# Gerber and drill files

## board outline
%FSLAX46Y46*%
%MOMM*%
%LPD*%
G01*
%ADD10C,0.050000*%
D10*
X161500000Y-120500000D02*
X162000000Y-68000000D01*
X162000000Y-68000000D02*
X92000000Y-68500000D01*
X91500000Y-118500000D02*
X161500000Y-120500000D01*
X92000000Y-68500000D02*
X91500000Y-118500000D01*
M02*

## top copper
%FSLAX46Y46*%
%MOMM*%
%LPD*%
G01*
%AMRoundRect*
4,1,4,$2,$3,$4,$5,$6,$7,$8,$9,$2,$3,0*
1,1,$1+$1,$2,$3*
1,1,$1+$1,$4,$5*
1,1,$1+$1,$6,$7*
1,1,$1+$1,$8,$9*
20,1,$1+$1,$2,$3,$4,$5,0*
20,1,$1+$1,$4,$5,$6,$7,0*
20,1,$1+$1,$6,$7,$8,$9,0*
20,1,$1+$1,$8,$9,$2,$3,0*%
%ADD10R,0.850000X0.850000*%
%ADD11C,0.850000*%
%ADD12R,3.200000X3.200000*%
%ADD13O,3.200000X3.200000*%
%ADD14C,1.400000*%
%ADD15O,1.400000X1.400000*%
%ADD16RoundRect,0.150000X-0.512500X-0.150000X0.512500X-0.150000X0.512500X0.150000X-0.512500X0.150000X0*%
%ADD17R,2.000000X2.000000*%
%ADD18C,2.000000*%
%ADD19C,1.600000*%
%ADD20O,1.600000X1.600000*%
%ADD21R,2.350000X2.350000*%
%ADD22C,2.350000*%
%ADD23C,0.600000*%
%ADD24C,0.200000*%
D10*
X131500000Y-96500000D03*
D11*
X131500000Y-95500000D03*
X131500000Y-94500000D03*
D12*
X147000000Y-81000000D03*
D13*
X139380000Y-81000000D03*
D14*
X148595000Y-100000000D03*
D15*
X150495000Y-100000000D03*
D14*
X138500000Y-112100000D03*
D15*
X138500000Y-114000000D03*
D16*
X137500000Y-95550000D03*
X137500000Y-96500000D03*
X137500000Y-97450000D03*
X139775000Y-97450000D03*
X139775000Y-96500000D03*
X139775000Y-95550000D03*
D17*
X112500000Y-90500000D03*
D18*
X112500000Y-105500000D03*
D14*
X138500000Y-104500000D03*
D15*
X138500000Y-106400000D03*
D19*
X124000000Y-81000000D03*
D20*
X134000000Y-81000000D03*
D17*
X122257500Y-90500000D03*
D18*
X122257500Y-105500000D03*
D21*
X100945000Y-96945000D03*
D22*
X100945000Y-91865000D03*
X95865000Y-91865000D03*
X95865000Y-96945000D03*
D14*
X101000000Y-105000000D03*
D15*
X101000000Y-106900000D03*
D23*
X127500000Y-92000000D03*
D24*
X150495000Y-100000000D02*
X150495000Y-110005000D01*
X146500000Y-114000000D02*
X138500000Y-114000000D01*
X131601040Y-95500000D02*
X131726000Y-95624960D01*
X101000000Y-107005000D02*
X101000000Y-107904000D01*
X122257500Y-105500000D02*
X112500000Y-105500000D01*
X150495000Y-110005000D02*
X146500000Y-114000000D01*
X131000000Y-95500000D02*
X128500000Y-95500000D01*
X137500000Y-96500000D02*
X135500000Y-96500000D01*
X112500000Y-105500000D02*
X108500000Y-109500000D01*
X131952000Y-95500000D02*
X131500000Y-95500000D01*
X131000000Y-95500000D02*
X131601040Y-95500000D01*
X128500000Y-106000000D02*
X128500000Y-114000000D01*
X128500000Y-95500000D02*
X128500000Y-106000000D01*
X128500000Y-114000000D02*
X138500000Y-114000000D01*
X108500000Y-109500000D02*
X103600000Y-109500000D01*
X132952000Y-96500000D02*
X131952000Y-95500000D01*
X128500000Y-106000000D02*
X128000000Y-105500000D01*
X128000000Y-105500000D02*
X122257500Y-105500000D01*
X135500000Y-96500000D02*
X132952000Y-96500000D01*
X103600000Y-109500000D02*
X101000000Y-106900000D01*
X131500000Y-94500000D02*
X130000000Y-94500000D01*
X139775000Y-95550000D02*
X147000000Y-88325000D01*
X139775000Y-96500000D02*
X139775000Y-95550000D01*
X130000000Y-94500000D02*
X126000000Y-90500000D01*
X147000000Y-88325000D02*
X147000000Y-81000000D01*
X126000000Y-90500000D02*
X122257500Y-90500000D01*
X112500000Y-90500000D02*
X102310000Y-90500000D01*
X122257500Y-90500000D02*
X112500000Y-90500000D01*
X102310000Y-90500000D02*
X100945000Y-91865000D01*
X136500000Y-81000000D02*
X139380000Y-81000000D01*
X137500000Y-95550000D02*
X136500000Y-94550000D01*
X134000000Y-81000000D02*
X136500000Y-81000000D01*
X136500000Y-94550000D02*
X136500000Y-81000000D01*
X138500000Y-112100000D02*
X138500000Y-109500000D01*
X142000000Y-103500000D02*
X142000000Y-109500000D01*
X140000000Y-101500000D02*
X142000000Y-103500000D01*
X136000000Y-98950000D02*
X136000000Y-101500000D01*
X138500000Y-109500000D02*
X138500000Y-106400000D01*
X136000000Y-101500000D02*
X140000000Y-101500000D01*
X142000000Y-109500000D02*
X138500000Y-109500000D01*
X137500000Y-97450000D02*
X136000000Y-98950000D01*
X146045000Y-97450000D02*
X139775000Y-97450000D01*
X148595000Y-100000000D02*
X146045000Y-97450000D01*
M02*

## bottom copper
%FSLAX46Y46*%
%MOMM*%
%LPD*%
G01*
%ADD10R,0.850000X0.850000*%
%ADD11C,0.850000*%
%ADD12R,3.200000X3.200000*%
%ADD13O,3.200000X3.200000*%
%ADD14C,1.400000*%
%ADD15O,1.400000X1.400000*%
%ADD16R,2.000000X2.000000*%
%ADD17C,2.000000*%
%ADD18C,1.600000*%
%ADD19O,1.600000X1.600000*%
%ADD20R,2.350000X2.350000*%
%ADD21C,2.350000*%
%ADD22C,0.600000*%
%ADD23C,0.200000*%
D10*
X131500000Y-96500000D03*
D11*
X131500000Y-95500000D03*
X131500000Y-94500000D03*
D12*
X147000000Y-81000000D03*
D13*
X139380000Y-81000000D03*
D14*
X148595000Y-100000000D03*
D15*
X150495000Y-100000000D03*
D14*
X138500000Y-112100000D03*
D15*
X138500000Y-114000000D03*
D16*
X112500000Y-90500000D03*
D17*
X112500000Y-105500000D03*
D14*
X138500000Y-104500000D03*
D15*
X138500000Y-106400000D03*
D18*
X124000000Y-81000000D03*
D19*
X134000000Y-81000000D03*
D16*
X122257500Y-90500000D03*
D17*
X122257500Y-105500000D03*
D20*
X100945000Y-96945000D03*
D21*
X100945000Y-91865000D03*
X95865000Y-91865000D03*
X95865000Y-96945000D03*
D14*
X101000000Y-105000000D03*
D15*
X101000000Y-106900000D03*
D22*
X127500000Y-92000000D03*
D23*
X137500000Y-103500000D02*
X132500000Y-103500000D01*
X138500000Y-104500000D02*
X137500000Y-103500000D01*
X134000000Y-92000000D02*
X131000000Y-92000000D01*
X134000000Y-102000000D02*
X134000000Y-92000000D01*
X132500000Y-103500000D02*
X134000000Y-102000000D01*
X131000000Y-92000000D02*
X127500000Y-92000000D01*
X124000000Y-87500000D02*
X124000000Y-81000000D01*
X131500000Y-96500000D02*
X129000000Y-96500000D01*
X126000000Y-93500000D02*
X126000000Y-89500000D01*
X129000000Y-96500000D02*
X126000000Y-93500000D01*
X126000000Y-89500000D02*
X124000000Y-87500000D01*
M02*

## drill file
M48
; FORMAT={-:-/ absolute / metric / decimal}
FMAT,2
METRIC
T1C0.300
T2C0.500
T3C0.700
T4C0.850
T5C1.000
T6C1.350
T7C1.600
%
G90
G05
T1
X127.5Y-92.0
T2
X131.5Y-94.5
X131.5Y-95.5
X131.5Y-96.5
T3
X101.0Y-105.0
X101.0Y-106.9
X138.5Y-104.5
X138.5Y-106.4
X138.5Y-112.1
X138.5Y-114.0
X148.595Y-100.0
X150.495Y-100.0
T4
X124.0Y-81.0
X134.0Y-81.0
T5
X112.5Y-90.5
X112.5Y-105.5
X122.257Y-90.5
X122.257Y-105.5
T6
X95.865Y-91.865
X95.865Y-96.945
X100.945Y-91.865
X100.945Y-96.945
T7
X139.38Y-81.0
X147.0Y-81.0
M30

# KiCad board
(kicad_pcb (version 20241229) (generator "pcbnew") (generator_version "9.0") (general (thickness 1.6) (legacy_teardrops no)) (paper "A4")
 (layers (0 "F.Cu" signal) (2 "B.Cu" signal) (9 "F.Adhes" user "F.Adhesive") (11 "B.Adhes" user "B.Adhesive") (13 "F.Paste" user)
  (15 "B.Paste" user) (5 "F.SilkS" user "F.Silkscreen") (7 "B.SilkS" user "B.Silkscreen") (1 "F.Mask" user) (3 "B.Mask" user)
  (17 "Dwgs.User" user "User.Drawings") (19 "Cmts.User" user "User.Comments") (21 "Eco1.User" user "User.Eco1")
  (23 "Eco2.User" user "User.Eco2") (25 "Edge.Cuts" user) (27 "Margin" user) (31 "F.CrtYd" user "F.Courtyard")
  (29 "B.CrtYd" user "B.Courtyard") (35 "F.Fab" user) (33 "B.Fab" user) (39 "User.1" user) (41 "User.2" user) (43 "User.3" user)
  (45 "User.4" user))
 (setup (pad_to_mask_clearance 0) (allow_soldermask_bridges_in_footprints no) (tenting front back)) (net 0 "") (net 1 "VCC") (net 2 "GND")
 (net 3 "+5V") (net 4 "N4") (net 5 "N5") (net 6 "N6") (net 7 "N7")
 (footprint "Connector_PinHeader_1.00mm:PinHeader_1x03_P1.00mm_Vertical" (layer "F.Cu") (at 131.5 96.5 180)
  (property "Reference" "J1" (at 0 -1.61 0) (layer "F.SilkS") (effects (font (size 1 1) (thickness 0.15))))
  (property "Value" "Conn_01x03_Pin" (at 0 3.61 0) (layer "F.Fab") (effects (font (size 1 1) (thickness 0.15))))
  (pad "1" thru_hole rect (at 0 0 180) (size 0.85 0.85) (drill 0.5) (layers "*.Cu" "*.Mask") (remove_unused_layers no) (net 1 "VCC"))
  (pad "2" thru_hole circle (at 0 1 180) (size 0.85 0.85) (drill 0.5) (layers "*.Cu" "*.Mask") (remove_unused_layers no) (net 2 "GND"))
  (pad "3" thru_hole circle (at 0 2 180) (size 0.85 0.85) (drill 0.5) (layers "*.Cu" "*.Mask") (remove_unused_layers no) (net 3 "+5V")))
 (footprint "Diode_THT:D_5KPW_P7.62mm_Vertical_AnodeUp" (layer "F.Cu") (at 147 81 180)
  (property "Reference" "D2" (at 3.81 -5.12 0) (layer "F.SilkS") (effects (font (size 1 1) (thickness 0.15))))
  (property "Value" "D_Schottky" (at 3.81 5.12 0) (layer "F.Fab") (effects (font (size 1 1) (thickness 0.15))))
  (pad "1" thru_hole rect (at 0 0 180) (size 3.2 3.2) (drill 1.6) (layers "*.Cu" "*.Mask") (remove_unused_layers no) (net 3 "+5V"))
  (pad "2" thru_hole oval (at 7.62 0 180) (size 3.2 3.2) (drill 1.6) (layers "*.Cu" "*.Mask") (remove_unused_layers no) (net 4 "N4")))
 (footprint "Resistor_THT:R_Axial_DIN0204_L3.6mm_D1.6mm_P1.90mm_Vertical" (layer "F.Cu") (at 148.595 100)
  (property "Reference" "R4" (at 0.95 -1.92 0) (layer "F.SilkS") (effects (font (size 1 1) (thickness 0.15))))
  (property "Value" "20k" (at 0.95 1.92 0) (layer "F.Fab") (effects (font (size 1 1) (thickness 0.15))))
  (pad "1" thru_hole circle (at 0 0) (size 1.4 1.4) (drill 0.7) (layers "*.Cu" "*.Mask") (remove_unused_layers no) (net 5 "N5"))
  (pad "2" thru_hole oval (at 1.9 0) (size 1.4 1.4) (drill 0.7) (layers "*.Cu" "*.Mask") (remove_unused_layers no) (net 2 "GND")))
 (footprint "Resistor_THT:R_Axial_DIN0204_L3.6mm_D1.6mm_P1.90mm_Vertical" (layer "F.Cu") (at 138.5 112.1 -90)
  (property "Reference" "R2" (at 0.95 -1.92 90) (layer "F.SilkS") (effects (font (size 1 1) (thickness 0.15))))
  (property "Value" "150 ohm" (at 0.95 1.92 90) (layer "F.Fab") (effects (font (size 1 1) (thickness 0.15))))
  (pad "1" thru_hole circle (at 0 0 270) (size 1.4 1.4) (drill 0.7) (layers "*.Cu" "*.Mask") (remove_unused_layers no) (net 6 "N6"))
  (pad "2" thru_hole oval (at 1.9 0 270) (size 1.4 1.4) (drill 0.7) (layers "*.Cu" "*.Mask") (remove_unused_layers no) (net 2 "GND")))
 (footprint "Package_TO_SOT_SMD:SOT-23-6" (layer "F.Cu") (at 138.6375 96.5)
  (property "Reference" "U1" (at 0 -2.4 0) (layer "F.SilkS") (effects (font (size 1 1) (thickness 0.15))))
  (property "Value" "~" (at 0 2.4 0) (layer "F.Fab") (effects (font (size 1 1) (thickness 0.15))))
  (pad "1" smd roundrect (at -1.1375 -0.95) (size 1.325 0.6) (layers "F.Cu" "F.Mask" "F.Paste") (roundrect_rratio 0.25) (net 4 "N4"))
  (pad "2" smd roundrect (at -1.1375 0) (size 1.325 0.6) (layers "F.Cu" "F.Mask" "F.Paste") (roundrect_rratio 0.25) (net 2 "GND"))
  (pad "3" smd roundrect (at -1.1375 0.95) (size 1.325 0.6) (layers "F.Cu" "F.Mask" "F.Paste") (roundrect_rratio 0.25) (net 6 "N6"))
  (pad "4" smd roundrect (at 1.1375 0.95) (size 1.325 0.6) (layers "F.Cu" "F.Mask" "F.Paste") (roundrect_rratio 0.25) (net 5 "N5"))
  (pad "5" smd roundrect (at 1.1375 0) (size 1.325 0.6) (layers "F.Cu" "F.Mask" "F.Paste") (roundrect_rratio 0.25) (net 3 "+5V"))
  (pad "6" smd roundrect (at 1.1375 -0.95) (size 1.325 0.6) (layers "F.Cu" "F.Mask" "F.Paste") (roundrect_rratio 0.25) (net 3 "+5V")))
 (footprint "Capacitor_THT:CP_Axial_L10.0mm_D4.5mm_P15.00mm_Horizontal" (layer "F.Cu") (at 112.5 90.5 -90)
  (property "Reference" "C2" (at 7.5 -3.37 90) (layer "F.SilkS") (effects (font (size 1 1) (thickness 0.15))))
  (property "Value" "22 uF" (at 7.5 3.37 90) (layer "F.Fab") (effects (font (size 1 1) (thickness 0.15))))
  (pad "1" thru_hole rect (at 0 0 270) (size 2 2) (drill 1) (layers "*.Cu" "*.Mask") (remove_unused_layers no) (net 3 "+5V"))
  (pad "2" thru_hole circle (at 15 0 270) (size 2 2) (drill 1) (layers "*.Cu" "*.Mask") (remove_unused_layers no) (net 2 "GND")))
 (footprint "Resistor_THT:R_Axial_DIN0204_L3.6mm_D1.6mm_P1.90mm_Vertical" (layer "F.Cu") (at 138.5 104.5 -90)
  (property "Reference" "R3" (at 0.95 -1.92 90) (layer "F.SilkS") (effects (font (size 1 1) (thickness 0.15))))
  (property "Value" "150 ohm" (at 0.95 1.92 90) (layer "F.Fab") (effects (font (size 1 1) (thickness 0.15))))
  (pad "1" thru_hole circle (at 0 0 270) (size 1.4 1.4) (drill 0.7) (layers "*.Cu" "*.Mask") (remove_unused_layers no) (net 3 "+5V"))
  (pad "2" thru_hole oval (at 1.9 0 270) (size 1.4 1.4) (drill 0.7) (layers "*.Cu" "*.Mask") (remove_unused_layers no) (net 6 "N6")))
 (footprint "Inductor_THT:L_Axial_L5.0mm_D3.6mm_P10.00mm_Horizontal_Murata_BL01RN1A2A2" (layer "F.Cu") (at 124 81)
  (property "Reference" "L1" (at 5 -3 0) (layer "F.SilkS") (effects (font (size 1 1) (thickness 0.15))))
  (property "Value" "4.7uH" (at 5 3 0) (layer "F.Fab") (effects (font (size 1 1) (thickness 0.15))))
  (pad "1" thru_hole circle (at 0 0) (size 1.6 1.6) (drill 0.85) (layers "*.Cu" "*.Mask") (remove_unused_layers no) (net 1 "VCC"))
  (pad "2" thru_hole oval (at 10 0) (size 1.6 1.6) (drill 0.85) (layers "*.Cu" "*.Mask") (remove_unused_layers no) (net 4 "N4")))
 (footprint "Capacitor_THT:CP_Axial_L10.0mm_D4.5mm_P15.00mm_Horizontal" (layer "F.Cu") (at 122.2575 90.5 -90)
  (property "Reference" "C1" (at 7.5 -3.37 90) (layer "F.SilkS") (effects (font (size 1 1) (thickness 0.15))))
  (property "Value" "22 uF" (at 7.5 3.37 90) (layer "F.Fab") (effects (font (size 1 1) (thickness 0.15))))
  (pad "1" thru_hole rect (at 0 0 270) (size 2 2) (drill 1) (layers "*.Cu" "*.Mask") (remove_unused_layers no) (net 3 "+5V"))
  (pad "2" thru_hole circle (at 15 0 270) (size 2 2) (drill 1) (layers "*.Cu" "*.Mask") (remove_unused_layers no) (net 2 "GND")))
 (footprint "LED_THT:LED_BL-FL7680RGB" (layer "F.Cu") (at 100.945 96.945 180)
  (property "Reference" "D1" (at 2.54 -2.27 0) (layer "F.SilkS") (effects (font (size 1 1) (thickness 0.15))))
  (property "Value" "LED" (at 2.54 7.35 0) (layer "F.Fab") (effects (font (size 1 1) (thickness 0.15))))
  (pad "1" thru_hole rect (at 0 0 180) (size 2.35 2.35) (drill 1.35) (layers "*.Cu" "*.Mask") (remove_unused_layers no) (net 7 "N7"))
  (pad "2" thru_hole circle (at 0 5.08 180) (size 2.35 2.35) (drill 1.35) (layers "*.Cu" "*.Mask") (remove_unused_layers no) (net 3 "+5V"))
  (pad "3" thru_hole circle (at 5.08 5.08 180) (size 2.35 2.35) (drill 1.35) (layers "*.Cu" "*.Mask") (remove_unused_layers no))
  (pad "4" thru_hole circle (at 5.08 0 180) (size 2.35 2.35) (drill 1.35) (layers "*.Cu" "*.Mask") (remove_unused_layers no)))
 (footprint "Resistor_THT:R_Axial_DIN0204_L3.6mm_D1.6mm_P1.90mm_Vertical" (layer "F.Cu") (at 101 105 -90)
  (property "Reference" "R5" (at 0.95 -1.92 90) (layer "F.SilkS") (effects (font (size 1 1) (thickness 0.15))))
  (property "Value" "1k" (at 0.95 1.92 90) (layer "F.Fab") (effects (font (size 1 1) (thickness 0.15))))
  (pad "1" thru_hole circle (at 0 0 270) (size 1.4 1.4) (drill 0.7) (layers "*.Cu" "*.Mask") (remove_unused_layers no) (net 7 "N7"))
  (pad "2" thru_hole oval (at 1.9 0 270) (size 1.4 1.4) (drill 0.7) (layers "*.Cu" "*.Mask") (remove_unused_layers no) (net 2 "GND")))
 (gr_line (start 161.5 120.5) (end 162 68) (stroke (width 0.05) (type default)) (layer "Edge.Cuts"))
 (gr_line (start 162 68) (end 92 68.5) (stroke (width 0.05) (type default)) (layer "Edge.Cuts"))
 (gr_line (start 91.5 118.5) (end 161.5 120.5) (stroke (width 0.05) (type default)) (layer "Edge.Cuts"))
 (gr_line (start 92 68.5) (end 91.5 118.5) (stroke (width 0.05) (type default)) (layer "Edge.Cuts"))
 (segment (start 150.495 100) (end 150.495 110.005) (width 0.2) (layer "F.Cu") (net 2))
 (segment (start 146.5 114) (end 138.5 114) (width 0.2) (layer "F.Cu") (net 2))
 (segment (start 131.60104 95.5) (end 131.726 95.62496) (width 0.2) (layer "F.Cu") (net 2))
 (segment (start 101 107.005) (end 101 107.904) (width 0.2) (layer "F.Cu") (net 2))
 (segment (start 122.2575 105.5) (end 112.5 105.5) (width 0.2) (layer "F.Cu") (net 2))
 (segment (start 150.495 110.005) (end 146.5 114) (width 0.2) (layer "F.Cu") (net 2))
 (segment (start 131 95.5) (end 128.5 95.5) (width 0.2) (layer "F.Cu") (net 2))
 (segment (start 137.5 96.5) (end 135.5 96.5) (width 0.2) (layer "F.Cu") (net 2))
 (segment (start 112.5 105.5) (end 108.5 109.5) (width 0.2) (layer "F.Cu") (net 2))
 (segment (start 131.952 95.5) (end 131.5 95.5) (width 0.2) (layer "F.Cu") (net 2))
 (segment (start 131 95.5) (end 131.60104 95.5) (width 0.2) (layer "F.Cu") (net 2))
 (segment (start 128.5 106) (end 128.5 114) (width 0.2) (layer "F.Cu") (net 2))
 (segment (start 128.5 95.5) (end 128.5 106) (width 0.2) (layer "F.Cu") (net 2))
 (segment (start 128.5 114) (end 138.5 114) (width 0.2) (layer "F.Cu") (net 2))
 (segment (start 108.5 109.5) (end 103.6 109.5) (width 0.2) (layer "F.Cu") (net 2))
 (segment (start 132.952 96.5) (end 131.952 95.5) (width 0.2) (layer "F.Cu") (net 2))
 (segment (start 128.5 106) (end 128 105.5) (width 0.2) (layer "F.Cu") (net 2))
 (segment (start 128 105.5) (end 122.2575 105.5) (width 0.2) (layer "F.Cu") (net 2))
 (segment (start 135.5 96.5) (end 132.952 96.5) (width 0.2) (layer "F.Cu") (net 2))
 (segment (start 103.6 109.5) (end 101 106.9) (width 0.2) (layer "F.Cu") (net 2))
 (segment (start 131.5 94.5) (end 130 94.5) (width 0.2) (layer "F.Cu") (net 3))
 (segment (start 139.775 95.55) (end 147 88.325) (width 0.2) (layer "F.Cu") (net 3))
 (segment (start 139.775 96.5) (end 139.775 95.55) (width 0.2) (layer "F.Cu") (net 3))
 (segment (start 130 94.5) (end 126 90.5) (width 0.2) (layer "F.Cu") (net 3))
 (segment (start 147 88.325) (end 147 81) (width 0.2) (layer "F.Cu") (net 3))
 (segment (start 126 90.5) (end 122.2575 90.5) (width 0.2) (layer "F.Cu") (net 3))
 (segment (start 112.5 90.5) (end 102.31 90.5) (width 0.2) (layer "F.Cu") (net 3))
 (segment (start 122.2575 90.5) (end 112.5 90.5) (width 0.2) (layer "F.Cu") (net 3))
 (segment (start 102.31 90.5) (end 100.945 91.865) (width 0.2) (layer "F.Cu") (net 3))
 (via (at 127.5 92) (size 0.6) (drill 0.3) (layers "F.Cu" "B.Cu") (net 3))
 (segment (start 137.5 103.5) (end 132.5 103.5) (width 0.2) (layer "B.Cu") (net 3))
 (segment (start 138.5 104.5) (end 137.5 103.5) (width 0.2) (layer "B.Cu") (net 3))
 (segment (start 134 92) (end 131 92) (width 0.2) (layer "B.Cu") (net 3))
 (segment (start 134 102) (end 134 92) (width 0.2) (layer "B.Cu") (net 3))
 (segment (start 132.5 103.5) (end 134 102) (width 0.2) (layer "B.Cu") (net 3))
 (segment (start 131 92) (end 127.5 92) (width 0.2) (layer "B.Cu") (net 3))
 (segment (start 136.5 81) (end 139.38 81) (width 0.2) (layer "F.Cu") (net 4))
 (segment (start 137.5 95.55) (end 136.5 94.55) (width 0.2) (layer "F.Cu") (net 4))
 (segment (start 134 81) (end 136.5 81) (width 0.2) (layer "F.Cu") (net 4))
 (segment (start 136.5 94.55) (end 136.5 81) (width 0.2) (layer "F.Cu") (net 4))
 (segment (start 124 87.5) (end 124 81) (width 0.2) (layer "B.Cu") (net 1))
 (segment (start 131.5 96.5) (end 129 96.5) (width 0.2) (layer "B.Cu") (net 1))
 (segment (start 126 93.5) (end 126 89.5) (width 0.2) (layer "B.Cu") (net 1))
 (segment (start 129 96.5) (end 126 93.5) (width 0.2) (layer "B.Cu") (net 1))
 (segment (start 126 89.5) (end 124 87.5) (width 0.2) (layer "B.Cu") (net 1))
 (segment (start 138.5 112.1) (end 138.5 109.5) (width 0.2) (layer "F.Cu") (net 6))
 (segment (start 142 103.5) (end 142 109.5) (width 0.2) (layer "F.Cu") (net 6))
 (segment (start 140 101.5) (end 142 103.5) (width 0.2) (layer "F.Cu") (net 6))
 (segment (start 136 98.95) (end 136 101.5) (width 0.2) (layer "F.Cu") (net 6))
 (segment (start 138.5 109.5) (end 138.5 106.4) (width 0.2) (layer "F.Cu") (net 6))
 (segment (start 136 101.5) (end 140 101.5) (width 0.2) (layer "F.Cu") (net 6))
 (segment (start 142 109.5) (end 138.5 109.5) (width 0.2) (layer "F.Cu") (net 6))
 (segment (start 137.5 97.45) (end 136 98.95) (width 0.2) (layer "F.Cu") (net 6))
 (segment (start 146.045 97.45) (end 139.775 97.45) (width 0.2) (layer "F.Cu") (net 5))
 (segment (start 148.595 100) (end 146.045 97.45) (width 0.2) (layer "F.Cu") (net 5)))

